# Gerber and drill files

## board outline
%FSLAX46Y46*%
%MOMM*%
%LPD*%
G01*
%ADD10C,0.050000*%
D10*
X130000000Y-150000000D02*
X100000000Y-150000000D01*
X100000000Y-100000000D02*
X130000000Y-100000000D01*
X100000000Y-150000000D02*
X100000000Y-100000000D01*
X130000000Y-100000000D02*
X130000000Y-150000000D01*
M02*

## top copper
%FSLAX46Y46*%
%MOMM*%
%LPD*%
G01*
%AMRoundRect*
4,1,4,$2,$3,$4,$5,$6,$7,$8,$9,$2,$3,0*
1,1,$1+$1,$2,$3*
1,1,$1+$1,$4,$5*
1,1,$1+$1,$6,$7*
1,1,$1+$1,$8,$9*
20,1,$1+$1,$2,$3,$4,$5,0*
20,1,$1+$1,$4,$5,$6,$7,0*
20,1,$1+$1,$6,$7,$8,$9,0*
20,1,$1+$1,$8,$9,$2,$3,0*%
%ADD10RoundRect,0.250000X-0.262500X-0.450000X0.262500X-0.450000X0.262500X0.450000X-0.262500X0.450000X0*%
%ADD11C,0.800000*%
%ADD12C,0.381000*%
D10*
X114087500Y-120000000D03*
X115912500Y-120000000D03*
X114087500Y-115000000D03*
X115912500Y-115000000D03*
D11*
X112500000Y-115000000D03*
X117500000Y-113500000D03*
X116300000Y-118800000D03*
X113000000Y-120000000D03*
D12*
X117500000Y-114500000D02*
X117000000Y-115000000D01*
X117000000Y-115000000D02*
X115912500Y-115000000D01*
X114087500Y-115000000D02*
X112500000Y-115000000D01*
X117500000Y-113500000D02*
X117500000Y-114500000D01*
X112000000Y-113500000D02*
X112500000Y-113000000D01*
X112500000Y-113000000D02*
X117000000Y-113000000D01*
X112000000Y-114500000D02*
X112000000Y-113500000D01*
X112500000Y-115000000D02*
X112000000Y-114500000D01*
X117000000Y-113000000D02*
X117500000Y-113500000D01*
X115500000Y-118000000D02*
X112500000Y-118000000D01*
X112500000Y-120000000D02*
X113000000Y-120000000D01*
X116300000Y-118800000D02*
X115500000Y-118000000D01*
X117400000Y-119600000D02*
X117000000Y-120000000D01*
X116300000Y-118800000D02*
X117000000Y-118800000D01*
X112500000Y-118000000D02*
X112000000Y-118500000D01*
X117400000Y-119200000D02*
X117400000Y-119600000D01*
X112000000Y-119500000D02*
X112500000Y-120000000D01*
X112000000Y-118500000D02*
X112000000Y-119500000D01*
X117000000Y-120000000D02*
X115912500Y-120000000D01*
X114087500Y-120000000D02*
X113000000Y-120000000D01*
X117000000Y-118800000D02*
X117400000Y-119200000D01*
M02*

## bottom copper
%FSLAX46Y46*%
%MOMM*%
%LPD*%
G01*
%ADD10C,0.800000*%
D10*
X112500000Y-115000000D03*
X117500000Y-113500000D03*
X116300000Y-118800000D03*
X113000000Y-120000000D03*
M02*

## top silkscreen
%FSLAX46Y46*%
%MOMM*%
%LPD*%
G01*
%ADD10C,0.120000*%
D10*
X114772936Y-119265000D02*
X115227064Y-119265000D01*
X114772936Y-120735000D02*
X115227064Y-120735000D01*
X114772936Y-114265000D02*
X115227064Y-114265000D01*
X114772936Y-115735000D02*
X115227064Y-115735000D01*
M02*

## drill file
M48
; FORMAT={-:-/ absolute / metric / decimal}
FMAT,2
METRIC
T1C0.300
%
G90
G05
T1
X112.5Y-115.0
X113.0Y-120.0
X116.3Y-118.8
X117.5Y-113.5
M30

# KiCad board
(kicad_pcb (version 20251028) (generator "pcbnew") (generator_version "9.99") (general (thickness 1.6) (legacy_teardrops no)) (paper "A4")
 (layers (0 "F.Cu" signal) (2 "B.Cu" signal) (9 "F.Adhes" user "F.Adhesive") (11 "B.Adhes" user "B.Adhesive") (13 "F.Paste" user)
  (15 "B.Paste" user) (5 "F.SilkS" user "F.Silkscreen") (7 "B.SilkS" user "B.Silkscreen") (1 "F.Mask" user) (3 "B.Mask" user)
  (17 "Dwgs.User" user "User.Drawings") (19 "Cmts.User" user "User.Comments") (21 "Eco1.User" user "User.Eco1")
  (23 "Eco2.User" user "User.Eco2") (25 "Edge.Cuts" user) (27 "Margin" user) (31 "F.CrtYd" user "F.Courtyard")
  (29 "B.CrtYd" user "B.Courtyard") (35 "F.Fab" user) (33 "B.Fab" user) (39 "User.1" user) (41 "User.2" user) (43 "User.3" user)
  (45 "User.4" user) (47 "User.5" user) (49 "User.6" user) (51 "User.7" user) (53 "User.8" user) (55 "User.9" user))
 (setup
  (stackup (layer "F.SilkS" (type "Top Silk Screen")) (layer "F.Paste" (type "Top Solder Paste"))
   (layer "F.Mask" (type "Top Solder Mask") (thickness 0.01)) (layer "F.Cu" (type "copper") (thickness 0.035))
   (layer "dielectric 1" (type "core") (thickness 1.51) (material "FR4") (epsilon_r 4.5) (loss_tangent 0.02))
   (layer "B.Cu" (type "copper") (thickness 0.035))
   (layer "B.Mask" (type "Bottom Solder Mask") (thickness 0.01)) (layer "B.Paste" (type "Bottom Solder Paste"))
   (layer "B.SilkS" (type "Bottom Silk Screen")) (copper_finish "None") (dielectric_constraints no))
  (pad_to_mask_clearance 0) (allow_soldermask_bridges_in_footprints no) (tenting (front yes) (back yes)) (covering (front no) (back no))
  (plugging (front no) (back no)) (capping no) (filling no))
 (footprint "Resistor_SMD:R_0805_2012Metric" (layer "F.Cu") (at 115 120)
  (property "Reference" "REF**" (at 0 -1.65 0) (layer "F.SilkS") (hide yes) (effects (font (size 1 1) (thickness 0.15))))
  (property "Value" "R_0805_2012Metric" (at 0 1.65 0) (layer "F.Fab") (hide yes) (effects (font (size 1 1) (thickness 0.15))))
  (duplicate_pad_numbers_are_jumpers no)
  (fp_line (start -0.227064 -0.735) (end 0.227064 -0.735) (stroke (width 0.12) (type solid)) (layer "F.SilkS"))
  (fp_line (start -0.227064 0.735) (end 0.227064 0.735) (stroke (width 0.12) (type solid)) (layer "F.SilkS"))
  (pad "1" smd roundrect (at -0.9125 0) (size 1.025 1.4) (layers "F.Cu" "F.Mask" "F.Paste") (roundrect_rratio 0.243902) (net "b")
   (tenting (front none) (back none)))
  (pad "2" smd roundrect (at 0.9125 0) (size 1.025 1.4) (layers "F.Cu" "F.Mask" "F.Paste") (roundrect_rratio 0.243902) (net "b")
   (tenting (front none) (back none))))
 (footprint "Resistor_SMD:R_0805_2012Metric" (layer "F.Cu") (at 115 115)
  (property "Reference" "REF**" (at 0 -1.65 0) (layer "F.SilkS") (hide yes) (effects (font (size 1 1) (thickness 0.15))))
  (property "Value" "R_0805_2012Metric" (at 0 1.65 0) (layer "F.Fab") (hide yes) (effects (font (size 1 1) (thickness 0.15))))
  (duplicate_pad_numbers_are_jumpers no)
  (fp_line (start -0.227064 -0.735) (end 0.227064 -0.735) (stroke (width 0.12) (type solid)) (layer "F.SilkS"))
  (fp_line (start -0.227064 0.735) (end 0.227064 0.735) (stroke (width 0.12) (type solid)) (layer "F.SilkS"))
  (pad "1" smd roundrect (at -0.9125 0) (size 1.025 1.4) (layers "F.Cu" "F.Mask" "F.Paste") (roundrect_rratio 0.243902) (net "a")
   (tenting (front none) (back none)))
  (pad "2" smd roundrect (at 0.9125 0) (size 1.025 1.4) (layers "F.Cu" "F.Mask" "F.Paste") (roundrect_rratio 0.243902) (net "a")
   (tenting (front none) (back none))))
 (gr_line (start 130 150) (end 100 150) (stroke (width 0.05) (type default)) (layer "Edge.Cuts"))
 (gr_line (start 100 100) (end 130 100) (stroke (width 0.05) (type default)) (layer "Edge.Cuts"))
 (gr_line (start 100 150) (end 100 100) (stroke (width 0.05) (type default)) (layer "Edge.Cuts"))
 (gr_line (start 130 100) (end 130 150) (stroke (width 0.05) (type default)) (layer "Edge.Cuts"))
 (segment (start 117.5 114.5) (end 117 115) (width 0.381) (layer "F.Cu") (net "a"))
 (segment (start 117 115) (end 115.9125 115) (width 0.381) (layer "F.Cu") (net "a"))
 (segment (start 114.0875 115) (end 112.5 115) (width 0.381) (layer "F.Cu") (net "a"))
 (segment (start 117.5 113.5) (end 117.5 114.5) (width 0.381) (layer "F.Cu") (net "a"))
 (segment (start 112 113.5) (end 112.5 113) (width 0.381) (layer "F.Cu") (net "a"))
 (segment (start 112.5 113) (end 117 113) (width 0.381) (layer "F.Cu") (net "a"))
 (segment (start 112 114.5) (end 112 113.5) (width 0.381) (layer "F.Cu") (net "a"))
 (segment (start 112.5 115) (end 112 114.5) (width 0.381) (layer "F.Cu") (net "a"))
 (segment (start 117 113) (end 117.5 113.5) (width 0.381) (layer "F.Cu") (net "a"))
 (via (at 112.5 115) (size 0.8) (drill 0.3) (layers "F.Cu" "B.Cu") (tenting (front none) (back none)) (capping none)
  (covering (front none) (back none)) (plugging (front none) (back none)) (filling none) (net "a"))
 (via (at 117.5 113.5) (size 0.8) (drill 0.3) (layers "F.Cu" "B.Cu") (tenting (front none) (back none)) (capping none)
  (covering (front none) (back none)) (plugging (front none) (back none)) (filling none) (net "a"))
 (segment (start 115.5 118) (end 112.5 118) (width 0.381) (layer "F.Cu") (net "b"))
 (segment (start 112.5 120) (end 113 120) (width 0.381) (layer "F.Cu") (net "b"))
 (segment (start 116.3 118.8) (end 115.5 118) (width 0.381) (layer "F.Cu") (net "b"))
 (segment (start 117.4 119.6) (end 117 120) (width 0.381) (layer "F.Cu") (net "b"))
 (segment (start 116.3 118.8) (end 117 118.8) (width 0.381) (layer "F.Cu") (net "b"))
 (segment (start 112.5 118) (end 112 118.5) (width 0.381) (layer "F.Cu") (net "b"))
 (segment (start 117.4 119.2) (end 117.4 119.6) (width 0.381) (layer "F.Cu") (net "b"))
 (segment (start 112 119.5) (end 112.5 120) (width 0.381) (layer "F.Cu") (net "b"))
 (segment (start 112 118.5) (end 112 119.5) (width 0.381) (layer "F.Cu") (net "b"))
 (segment (start 117 120) (end 115.9125 120) (width 0.381) (layer "F.Cu") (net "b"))
 (segment (start 114.0875 120) (end 113 120) (width 0.381) (layer "F.Cu") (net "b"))
 (segment (start 117 118.8) (end 117.4 119.2) (width 0.381) (layer "F.Cu") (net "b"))
 (via (at 116.3 118.8) (size 0.8) (drill 0.3) (layers "F.Cu" "B.Cu") (tenting (front none) (back none)) (capping none)
  (covering (front none) (back none)) (plugging (front none) (back none)) (filling none) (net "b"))
 (via (at 113 120) (size 0.8) (drill 0.3) (layers "F.Cu" "B.Cu") (tenting (front none) (back none)) (capping none)
  (covering (front none) (back none)) (plugging (front none) (back none)) (filling none) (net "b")))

